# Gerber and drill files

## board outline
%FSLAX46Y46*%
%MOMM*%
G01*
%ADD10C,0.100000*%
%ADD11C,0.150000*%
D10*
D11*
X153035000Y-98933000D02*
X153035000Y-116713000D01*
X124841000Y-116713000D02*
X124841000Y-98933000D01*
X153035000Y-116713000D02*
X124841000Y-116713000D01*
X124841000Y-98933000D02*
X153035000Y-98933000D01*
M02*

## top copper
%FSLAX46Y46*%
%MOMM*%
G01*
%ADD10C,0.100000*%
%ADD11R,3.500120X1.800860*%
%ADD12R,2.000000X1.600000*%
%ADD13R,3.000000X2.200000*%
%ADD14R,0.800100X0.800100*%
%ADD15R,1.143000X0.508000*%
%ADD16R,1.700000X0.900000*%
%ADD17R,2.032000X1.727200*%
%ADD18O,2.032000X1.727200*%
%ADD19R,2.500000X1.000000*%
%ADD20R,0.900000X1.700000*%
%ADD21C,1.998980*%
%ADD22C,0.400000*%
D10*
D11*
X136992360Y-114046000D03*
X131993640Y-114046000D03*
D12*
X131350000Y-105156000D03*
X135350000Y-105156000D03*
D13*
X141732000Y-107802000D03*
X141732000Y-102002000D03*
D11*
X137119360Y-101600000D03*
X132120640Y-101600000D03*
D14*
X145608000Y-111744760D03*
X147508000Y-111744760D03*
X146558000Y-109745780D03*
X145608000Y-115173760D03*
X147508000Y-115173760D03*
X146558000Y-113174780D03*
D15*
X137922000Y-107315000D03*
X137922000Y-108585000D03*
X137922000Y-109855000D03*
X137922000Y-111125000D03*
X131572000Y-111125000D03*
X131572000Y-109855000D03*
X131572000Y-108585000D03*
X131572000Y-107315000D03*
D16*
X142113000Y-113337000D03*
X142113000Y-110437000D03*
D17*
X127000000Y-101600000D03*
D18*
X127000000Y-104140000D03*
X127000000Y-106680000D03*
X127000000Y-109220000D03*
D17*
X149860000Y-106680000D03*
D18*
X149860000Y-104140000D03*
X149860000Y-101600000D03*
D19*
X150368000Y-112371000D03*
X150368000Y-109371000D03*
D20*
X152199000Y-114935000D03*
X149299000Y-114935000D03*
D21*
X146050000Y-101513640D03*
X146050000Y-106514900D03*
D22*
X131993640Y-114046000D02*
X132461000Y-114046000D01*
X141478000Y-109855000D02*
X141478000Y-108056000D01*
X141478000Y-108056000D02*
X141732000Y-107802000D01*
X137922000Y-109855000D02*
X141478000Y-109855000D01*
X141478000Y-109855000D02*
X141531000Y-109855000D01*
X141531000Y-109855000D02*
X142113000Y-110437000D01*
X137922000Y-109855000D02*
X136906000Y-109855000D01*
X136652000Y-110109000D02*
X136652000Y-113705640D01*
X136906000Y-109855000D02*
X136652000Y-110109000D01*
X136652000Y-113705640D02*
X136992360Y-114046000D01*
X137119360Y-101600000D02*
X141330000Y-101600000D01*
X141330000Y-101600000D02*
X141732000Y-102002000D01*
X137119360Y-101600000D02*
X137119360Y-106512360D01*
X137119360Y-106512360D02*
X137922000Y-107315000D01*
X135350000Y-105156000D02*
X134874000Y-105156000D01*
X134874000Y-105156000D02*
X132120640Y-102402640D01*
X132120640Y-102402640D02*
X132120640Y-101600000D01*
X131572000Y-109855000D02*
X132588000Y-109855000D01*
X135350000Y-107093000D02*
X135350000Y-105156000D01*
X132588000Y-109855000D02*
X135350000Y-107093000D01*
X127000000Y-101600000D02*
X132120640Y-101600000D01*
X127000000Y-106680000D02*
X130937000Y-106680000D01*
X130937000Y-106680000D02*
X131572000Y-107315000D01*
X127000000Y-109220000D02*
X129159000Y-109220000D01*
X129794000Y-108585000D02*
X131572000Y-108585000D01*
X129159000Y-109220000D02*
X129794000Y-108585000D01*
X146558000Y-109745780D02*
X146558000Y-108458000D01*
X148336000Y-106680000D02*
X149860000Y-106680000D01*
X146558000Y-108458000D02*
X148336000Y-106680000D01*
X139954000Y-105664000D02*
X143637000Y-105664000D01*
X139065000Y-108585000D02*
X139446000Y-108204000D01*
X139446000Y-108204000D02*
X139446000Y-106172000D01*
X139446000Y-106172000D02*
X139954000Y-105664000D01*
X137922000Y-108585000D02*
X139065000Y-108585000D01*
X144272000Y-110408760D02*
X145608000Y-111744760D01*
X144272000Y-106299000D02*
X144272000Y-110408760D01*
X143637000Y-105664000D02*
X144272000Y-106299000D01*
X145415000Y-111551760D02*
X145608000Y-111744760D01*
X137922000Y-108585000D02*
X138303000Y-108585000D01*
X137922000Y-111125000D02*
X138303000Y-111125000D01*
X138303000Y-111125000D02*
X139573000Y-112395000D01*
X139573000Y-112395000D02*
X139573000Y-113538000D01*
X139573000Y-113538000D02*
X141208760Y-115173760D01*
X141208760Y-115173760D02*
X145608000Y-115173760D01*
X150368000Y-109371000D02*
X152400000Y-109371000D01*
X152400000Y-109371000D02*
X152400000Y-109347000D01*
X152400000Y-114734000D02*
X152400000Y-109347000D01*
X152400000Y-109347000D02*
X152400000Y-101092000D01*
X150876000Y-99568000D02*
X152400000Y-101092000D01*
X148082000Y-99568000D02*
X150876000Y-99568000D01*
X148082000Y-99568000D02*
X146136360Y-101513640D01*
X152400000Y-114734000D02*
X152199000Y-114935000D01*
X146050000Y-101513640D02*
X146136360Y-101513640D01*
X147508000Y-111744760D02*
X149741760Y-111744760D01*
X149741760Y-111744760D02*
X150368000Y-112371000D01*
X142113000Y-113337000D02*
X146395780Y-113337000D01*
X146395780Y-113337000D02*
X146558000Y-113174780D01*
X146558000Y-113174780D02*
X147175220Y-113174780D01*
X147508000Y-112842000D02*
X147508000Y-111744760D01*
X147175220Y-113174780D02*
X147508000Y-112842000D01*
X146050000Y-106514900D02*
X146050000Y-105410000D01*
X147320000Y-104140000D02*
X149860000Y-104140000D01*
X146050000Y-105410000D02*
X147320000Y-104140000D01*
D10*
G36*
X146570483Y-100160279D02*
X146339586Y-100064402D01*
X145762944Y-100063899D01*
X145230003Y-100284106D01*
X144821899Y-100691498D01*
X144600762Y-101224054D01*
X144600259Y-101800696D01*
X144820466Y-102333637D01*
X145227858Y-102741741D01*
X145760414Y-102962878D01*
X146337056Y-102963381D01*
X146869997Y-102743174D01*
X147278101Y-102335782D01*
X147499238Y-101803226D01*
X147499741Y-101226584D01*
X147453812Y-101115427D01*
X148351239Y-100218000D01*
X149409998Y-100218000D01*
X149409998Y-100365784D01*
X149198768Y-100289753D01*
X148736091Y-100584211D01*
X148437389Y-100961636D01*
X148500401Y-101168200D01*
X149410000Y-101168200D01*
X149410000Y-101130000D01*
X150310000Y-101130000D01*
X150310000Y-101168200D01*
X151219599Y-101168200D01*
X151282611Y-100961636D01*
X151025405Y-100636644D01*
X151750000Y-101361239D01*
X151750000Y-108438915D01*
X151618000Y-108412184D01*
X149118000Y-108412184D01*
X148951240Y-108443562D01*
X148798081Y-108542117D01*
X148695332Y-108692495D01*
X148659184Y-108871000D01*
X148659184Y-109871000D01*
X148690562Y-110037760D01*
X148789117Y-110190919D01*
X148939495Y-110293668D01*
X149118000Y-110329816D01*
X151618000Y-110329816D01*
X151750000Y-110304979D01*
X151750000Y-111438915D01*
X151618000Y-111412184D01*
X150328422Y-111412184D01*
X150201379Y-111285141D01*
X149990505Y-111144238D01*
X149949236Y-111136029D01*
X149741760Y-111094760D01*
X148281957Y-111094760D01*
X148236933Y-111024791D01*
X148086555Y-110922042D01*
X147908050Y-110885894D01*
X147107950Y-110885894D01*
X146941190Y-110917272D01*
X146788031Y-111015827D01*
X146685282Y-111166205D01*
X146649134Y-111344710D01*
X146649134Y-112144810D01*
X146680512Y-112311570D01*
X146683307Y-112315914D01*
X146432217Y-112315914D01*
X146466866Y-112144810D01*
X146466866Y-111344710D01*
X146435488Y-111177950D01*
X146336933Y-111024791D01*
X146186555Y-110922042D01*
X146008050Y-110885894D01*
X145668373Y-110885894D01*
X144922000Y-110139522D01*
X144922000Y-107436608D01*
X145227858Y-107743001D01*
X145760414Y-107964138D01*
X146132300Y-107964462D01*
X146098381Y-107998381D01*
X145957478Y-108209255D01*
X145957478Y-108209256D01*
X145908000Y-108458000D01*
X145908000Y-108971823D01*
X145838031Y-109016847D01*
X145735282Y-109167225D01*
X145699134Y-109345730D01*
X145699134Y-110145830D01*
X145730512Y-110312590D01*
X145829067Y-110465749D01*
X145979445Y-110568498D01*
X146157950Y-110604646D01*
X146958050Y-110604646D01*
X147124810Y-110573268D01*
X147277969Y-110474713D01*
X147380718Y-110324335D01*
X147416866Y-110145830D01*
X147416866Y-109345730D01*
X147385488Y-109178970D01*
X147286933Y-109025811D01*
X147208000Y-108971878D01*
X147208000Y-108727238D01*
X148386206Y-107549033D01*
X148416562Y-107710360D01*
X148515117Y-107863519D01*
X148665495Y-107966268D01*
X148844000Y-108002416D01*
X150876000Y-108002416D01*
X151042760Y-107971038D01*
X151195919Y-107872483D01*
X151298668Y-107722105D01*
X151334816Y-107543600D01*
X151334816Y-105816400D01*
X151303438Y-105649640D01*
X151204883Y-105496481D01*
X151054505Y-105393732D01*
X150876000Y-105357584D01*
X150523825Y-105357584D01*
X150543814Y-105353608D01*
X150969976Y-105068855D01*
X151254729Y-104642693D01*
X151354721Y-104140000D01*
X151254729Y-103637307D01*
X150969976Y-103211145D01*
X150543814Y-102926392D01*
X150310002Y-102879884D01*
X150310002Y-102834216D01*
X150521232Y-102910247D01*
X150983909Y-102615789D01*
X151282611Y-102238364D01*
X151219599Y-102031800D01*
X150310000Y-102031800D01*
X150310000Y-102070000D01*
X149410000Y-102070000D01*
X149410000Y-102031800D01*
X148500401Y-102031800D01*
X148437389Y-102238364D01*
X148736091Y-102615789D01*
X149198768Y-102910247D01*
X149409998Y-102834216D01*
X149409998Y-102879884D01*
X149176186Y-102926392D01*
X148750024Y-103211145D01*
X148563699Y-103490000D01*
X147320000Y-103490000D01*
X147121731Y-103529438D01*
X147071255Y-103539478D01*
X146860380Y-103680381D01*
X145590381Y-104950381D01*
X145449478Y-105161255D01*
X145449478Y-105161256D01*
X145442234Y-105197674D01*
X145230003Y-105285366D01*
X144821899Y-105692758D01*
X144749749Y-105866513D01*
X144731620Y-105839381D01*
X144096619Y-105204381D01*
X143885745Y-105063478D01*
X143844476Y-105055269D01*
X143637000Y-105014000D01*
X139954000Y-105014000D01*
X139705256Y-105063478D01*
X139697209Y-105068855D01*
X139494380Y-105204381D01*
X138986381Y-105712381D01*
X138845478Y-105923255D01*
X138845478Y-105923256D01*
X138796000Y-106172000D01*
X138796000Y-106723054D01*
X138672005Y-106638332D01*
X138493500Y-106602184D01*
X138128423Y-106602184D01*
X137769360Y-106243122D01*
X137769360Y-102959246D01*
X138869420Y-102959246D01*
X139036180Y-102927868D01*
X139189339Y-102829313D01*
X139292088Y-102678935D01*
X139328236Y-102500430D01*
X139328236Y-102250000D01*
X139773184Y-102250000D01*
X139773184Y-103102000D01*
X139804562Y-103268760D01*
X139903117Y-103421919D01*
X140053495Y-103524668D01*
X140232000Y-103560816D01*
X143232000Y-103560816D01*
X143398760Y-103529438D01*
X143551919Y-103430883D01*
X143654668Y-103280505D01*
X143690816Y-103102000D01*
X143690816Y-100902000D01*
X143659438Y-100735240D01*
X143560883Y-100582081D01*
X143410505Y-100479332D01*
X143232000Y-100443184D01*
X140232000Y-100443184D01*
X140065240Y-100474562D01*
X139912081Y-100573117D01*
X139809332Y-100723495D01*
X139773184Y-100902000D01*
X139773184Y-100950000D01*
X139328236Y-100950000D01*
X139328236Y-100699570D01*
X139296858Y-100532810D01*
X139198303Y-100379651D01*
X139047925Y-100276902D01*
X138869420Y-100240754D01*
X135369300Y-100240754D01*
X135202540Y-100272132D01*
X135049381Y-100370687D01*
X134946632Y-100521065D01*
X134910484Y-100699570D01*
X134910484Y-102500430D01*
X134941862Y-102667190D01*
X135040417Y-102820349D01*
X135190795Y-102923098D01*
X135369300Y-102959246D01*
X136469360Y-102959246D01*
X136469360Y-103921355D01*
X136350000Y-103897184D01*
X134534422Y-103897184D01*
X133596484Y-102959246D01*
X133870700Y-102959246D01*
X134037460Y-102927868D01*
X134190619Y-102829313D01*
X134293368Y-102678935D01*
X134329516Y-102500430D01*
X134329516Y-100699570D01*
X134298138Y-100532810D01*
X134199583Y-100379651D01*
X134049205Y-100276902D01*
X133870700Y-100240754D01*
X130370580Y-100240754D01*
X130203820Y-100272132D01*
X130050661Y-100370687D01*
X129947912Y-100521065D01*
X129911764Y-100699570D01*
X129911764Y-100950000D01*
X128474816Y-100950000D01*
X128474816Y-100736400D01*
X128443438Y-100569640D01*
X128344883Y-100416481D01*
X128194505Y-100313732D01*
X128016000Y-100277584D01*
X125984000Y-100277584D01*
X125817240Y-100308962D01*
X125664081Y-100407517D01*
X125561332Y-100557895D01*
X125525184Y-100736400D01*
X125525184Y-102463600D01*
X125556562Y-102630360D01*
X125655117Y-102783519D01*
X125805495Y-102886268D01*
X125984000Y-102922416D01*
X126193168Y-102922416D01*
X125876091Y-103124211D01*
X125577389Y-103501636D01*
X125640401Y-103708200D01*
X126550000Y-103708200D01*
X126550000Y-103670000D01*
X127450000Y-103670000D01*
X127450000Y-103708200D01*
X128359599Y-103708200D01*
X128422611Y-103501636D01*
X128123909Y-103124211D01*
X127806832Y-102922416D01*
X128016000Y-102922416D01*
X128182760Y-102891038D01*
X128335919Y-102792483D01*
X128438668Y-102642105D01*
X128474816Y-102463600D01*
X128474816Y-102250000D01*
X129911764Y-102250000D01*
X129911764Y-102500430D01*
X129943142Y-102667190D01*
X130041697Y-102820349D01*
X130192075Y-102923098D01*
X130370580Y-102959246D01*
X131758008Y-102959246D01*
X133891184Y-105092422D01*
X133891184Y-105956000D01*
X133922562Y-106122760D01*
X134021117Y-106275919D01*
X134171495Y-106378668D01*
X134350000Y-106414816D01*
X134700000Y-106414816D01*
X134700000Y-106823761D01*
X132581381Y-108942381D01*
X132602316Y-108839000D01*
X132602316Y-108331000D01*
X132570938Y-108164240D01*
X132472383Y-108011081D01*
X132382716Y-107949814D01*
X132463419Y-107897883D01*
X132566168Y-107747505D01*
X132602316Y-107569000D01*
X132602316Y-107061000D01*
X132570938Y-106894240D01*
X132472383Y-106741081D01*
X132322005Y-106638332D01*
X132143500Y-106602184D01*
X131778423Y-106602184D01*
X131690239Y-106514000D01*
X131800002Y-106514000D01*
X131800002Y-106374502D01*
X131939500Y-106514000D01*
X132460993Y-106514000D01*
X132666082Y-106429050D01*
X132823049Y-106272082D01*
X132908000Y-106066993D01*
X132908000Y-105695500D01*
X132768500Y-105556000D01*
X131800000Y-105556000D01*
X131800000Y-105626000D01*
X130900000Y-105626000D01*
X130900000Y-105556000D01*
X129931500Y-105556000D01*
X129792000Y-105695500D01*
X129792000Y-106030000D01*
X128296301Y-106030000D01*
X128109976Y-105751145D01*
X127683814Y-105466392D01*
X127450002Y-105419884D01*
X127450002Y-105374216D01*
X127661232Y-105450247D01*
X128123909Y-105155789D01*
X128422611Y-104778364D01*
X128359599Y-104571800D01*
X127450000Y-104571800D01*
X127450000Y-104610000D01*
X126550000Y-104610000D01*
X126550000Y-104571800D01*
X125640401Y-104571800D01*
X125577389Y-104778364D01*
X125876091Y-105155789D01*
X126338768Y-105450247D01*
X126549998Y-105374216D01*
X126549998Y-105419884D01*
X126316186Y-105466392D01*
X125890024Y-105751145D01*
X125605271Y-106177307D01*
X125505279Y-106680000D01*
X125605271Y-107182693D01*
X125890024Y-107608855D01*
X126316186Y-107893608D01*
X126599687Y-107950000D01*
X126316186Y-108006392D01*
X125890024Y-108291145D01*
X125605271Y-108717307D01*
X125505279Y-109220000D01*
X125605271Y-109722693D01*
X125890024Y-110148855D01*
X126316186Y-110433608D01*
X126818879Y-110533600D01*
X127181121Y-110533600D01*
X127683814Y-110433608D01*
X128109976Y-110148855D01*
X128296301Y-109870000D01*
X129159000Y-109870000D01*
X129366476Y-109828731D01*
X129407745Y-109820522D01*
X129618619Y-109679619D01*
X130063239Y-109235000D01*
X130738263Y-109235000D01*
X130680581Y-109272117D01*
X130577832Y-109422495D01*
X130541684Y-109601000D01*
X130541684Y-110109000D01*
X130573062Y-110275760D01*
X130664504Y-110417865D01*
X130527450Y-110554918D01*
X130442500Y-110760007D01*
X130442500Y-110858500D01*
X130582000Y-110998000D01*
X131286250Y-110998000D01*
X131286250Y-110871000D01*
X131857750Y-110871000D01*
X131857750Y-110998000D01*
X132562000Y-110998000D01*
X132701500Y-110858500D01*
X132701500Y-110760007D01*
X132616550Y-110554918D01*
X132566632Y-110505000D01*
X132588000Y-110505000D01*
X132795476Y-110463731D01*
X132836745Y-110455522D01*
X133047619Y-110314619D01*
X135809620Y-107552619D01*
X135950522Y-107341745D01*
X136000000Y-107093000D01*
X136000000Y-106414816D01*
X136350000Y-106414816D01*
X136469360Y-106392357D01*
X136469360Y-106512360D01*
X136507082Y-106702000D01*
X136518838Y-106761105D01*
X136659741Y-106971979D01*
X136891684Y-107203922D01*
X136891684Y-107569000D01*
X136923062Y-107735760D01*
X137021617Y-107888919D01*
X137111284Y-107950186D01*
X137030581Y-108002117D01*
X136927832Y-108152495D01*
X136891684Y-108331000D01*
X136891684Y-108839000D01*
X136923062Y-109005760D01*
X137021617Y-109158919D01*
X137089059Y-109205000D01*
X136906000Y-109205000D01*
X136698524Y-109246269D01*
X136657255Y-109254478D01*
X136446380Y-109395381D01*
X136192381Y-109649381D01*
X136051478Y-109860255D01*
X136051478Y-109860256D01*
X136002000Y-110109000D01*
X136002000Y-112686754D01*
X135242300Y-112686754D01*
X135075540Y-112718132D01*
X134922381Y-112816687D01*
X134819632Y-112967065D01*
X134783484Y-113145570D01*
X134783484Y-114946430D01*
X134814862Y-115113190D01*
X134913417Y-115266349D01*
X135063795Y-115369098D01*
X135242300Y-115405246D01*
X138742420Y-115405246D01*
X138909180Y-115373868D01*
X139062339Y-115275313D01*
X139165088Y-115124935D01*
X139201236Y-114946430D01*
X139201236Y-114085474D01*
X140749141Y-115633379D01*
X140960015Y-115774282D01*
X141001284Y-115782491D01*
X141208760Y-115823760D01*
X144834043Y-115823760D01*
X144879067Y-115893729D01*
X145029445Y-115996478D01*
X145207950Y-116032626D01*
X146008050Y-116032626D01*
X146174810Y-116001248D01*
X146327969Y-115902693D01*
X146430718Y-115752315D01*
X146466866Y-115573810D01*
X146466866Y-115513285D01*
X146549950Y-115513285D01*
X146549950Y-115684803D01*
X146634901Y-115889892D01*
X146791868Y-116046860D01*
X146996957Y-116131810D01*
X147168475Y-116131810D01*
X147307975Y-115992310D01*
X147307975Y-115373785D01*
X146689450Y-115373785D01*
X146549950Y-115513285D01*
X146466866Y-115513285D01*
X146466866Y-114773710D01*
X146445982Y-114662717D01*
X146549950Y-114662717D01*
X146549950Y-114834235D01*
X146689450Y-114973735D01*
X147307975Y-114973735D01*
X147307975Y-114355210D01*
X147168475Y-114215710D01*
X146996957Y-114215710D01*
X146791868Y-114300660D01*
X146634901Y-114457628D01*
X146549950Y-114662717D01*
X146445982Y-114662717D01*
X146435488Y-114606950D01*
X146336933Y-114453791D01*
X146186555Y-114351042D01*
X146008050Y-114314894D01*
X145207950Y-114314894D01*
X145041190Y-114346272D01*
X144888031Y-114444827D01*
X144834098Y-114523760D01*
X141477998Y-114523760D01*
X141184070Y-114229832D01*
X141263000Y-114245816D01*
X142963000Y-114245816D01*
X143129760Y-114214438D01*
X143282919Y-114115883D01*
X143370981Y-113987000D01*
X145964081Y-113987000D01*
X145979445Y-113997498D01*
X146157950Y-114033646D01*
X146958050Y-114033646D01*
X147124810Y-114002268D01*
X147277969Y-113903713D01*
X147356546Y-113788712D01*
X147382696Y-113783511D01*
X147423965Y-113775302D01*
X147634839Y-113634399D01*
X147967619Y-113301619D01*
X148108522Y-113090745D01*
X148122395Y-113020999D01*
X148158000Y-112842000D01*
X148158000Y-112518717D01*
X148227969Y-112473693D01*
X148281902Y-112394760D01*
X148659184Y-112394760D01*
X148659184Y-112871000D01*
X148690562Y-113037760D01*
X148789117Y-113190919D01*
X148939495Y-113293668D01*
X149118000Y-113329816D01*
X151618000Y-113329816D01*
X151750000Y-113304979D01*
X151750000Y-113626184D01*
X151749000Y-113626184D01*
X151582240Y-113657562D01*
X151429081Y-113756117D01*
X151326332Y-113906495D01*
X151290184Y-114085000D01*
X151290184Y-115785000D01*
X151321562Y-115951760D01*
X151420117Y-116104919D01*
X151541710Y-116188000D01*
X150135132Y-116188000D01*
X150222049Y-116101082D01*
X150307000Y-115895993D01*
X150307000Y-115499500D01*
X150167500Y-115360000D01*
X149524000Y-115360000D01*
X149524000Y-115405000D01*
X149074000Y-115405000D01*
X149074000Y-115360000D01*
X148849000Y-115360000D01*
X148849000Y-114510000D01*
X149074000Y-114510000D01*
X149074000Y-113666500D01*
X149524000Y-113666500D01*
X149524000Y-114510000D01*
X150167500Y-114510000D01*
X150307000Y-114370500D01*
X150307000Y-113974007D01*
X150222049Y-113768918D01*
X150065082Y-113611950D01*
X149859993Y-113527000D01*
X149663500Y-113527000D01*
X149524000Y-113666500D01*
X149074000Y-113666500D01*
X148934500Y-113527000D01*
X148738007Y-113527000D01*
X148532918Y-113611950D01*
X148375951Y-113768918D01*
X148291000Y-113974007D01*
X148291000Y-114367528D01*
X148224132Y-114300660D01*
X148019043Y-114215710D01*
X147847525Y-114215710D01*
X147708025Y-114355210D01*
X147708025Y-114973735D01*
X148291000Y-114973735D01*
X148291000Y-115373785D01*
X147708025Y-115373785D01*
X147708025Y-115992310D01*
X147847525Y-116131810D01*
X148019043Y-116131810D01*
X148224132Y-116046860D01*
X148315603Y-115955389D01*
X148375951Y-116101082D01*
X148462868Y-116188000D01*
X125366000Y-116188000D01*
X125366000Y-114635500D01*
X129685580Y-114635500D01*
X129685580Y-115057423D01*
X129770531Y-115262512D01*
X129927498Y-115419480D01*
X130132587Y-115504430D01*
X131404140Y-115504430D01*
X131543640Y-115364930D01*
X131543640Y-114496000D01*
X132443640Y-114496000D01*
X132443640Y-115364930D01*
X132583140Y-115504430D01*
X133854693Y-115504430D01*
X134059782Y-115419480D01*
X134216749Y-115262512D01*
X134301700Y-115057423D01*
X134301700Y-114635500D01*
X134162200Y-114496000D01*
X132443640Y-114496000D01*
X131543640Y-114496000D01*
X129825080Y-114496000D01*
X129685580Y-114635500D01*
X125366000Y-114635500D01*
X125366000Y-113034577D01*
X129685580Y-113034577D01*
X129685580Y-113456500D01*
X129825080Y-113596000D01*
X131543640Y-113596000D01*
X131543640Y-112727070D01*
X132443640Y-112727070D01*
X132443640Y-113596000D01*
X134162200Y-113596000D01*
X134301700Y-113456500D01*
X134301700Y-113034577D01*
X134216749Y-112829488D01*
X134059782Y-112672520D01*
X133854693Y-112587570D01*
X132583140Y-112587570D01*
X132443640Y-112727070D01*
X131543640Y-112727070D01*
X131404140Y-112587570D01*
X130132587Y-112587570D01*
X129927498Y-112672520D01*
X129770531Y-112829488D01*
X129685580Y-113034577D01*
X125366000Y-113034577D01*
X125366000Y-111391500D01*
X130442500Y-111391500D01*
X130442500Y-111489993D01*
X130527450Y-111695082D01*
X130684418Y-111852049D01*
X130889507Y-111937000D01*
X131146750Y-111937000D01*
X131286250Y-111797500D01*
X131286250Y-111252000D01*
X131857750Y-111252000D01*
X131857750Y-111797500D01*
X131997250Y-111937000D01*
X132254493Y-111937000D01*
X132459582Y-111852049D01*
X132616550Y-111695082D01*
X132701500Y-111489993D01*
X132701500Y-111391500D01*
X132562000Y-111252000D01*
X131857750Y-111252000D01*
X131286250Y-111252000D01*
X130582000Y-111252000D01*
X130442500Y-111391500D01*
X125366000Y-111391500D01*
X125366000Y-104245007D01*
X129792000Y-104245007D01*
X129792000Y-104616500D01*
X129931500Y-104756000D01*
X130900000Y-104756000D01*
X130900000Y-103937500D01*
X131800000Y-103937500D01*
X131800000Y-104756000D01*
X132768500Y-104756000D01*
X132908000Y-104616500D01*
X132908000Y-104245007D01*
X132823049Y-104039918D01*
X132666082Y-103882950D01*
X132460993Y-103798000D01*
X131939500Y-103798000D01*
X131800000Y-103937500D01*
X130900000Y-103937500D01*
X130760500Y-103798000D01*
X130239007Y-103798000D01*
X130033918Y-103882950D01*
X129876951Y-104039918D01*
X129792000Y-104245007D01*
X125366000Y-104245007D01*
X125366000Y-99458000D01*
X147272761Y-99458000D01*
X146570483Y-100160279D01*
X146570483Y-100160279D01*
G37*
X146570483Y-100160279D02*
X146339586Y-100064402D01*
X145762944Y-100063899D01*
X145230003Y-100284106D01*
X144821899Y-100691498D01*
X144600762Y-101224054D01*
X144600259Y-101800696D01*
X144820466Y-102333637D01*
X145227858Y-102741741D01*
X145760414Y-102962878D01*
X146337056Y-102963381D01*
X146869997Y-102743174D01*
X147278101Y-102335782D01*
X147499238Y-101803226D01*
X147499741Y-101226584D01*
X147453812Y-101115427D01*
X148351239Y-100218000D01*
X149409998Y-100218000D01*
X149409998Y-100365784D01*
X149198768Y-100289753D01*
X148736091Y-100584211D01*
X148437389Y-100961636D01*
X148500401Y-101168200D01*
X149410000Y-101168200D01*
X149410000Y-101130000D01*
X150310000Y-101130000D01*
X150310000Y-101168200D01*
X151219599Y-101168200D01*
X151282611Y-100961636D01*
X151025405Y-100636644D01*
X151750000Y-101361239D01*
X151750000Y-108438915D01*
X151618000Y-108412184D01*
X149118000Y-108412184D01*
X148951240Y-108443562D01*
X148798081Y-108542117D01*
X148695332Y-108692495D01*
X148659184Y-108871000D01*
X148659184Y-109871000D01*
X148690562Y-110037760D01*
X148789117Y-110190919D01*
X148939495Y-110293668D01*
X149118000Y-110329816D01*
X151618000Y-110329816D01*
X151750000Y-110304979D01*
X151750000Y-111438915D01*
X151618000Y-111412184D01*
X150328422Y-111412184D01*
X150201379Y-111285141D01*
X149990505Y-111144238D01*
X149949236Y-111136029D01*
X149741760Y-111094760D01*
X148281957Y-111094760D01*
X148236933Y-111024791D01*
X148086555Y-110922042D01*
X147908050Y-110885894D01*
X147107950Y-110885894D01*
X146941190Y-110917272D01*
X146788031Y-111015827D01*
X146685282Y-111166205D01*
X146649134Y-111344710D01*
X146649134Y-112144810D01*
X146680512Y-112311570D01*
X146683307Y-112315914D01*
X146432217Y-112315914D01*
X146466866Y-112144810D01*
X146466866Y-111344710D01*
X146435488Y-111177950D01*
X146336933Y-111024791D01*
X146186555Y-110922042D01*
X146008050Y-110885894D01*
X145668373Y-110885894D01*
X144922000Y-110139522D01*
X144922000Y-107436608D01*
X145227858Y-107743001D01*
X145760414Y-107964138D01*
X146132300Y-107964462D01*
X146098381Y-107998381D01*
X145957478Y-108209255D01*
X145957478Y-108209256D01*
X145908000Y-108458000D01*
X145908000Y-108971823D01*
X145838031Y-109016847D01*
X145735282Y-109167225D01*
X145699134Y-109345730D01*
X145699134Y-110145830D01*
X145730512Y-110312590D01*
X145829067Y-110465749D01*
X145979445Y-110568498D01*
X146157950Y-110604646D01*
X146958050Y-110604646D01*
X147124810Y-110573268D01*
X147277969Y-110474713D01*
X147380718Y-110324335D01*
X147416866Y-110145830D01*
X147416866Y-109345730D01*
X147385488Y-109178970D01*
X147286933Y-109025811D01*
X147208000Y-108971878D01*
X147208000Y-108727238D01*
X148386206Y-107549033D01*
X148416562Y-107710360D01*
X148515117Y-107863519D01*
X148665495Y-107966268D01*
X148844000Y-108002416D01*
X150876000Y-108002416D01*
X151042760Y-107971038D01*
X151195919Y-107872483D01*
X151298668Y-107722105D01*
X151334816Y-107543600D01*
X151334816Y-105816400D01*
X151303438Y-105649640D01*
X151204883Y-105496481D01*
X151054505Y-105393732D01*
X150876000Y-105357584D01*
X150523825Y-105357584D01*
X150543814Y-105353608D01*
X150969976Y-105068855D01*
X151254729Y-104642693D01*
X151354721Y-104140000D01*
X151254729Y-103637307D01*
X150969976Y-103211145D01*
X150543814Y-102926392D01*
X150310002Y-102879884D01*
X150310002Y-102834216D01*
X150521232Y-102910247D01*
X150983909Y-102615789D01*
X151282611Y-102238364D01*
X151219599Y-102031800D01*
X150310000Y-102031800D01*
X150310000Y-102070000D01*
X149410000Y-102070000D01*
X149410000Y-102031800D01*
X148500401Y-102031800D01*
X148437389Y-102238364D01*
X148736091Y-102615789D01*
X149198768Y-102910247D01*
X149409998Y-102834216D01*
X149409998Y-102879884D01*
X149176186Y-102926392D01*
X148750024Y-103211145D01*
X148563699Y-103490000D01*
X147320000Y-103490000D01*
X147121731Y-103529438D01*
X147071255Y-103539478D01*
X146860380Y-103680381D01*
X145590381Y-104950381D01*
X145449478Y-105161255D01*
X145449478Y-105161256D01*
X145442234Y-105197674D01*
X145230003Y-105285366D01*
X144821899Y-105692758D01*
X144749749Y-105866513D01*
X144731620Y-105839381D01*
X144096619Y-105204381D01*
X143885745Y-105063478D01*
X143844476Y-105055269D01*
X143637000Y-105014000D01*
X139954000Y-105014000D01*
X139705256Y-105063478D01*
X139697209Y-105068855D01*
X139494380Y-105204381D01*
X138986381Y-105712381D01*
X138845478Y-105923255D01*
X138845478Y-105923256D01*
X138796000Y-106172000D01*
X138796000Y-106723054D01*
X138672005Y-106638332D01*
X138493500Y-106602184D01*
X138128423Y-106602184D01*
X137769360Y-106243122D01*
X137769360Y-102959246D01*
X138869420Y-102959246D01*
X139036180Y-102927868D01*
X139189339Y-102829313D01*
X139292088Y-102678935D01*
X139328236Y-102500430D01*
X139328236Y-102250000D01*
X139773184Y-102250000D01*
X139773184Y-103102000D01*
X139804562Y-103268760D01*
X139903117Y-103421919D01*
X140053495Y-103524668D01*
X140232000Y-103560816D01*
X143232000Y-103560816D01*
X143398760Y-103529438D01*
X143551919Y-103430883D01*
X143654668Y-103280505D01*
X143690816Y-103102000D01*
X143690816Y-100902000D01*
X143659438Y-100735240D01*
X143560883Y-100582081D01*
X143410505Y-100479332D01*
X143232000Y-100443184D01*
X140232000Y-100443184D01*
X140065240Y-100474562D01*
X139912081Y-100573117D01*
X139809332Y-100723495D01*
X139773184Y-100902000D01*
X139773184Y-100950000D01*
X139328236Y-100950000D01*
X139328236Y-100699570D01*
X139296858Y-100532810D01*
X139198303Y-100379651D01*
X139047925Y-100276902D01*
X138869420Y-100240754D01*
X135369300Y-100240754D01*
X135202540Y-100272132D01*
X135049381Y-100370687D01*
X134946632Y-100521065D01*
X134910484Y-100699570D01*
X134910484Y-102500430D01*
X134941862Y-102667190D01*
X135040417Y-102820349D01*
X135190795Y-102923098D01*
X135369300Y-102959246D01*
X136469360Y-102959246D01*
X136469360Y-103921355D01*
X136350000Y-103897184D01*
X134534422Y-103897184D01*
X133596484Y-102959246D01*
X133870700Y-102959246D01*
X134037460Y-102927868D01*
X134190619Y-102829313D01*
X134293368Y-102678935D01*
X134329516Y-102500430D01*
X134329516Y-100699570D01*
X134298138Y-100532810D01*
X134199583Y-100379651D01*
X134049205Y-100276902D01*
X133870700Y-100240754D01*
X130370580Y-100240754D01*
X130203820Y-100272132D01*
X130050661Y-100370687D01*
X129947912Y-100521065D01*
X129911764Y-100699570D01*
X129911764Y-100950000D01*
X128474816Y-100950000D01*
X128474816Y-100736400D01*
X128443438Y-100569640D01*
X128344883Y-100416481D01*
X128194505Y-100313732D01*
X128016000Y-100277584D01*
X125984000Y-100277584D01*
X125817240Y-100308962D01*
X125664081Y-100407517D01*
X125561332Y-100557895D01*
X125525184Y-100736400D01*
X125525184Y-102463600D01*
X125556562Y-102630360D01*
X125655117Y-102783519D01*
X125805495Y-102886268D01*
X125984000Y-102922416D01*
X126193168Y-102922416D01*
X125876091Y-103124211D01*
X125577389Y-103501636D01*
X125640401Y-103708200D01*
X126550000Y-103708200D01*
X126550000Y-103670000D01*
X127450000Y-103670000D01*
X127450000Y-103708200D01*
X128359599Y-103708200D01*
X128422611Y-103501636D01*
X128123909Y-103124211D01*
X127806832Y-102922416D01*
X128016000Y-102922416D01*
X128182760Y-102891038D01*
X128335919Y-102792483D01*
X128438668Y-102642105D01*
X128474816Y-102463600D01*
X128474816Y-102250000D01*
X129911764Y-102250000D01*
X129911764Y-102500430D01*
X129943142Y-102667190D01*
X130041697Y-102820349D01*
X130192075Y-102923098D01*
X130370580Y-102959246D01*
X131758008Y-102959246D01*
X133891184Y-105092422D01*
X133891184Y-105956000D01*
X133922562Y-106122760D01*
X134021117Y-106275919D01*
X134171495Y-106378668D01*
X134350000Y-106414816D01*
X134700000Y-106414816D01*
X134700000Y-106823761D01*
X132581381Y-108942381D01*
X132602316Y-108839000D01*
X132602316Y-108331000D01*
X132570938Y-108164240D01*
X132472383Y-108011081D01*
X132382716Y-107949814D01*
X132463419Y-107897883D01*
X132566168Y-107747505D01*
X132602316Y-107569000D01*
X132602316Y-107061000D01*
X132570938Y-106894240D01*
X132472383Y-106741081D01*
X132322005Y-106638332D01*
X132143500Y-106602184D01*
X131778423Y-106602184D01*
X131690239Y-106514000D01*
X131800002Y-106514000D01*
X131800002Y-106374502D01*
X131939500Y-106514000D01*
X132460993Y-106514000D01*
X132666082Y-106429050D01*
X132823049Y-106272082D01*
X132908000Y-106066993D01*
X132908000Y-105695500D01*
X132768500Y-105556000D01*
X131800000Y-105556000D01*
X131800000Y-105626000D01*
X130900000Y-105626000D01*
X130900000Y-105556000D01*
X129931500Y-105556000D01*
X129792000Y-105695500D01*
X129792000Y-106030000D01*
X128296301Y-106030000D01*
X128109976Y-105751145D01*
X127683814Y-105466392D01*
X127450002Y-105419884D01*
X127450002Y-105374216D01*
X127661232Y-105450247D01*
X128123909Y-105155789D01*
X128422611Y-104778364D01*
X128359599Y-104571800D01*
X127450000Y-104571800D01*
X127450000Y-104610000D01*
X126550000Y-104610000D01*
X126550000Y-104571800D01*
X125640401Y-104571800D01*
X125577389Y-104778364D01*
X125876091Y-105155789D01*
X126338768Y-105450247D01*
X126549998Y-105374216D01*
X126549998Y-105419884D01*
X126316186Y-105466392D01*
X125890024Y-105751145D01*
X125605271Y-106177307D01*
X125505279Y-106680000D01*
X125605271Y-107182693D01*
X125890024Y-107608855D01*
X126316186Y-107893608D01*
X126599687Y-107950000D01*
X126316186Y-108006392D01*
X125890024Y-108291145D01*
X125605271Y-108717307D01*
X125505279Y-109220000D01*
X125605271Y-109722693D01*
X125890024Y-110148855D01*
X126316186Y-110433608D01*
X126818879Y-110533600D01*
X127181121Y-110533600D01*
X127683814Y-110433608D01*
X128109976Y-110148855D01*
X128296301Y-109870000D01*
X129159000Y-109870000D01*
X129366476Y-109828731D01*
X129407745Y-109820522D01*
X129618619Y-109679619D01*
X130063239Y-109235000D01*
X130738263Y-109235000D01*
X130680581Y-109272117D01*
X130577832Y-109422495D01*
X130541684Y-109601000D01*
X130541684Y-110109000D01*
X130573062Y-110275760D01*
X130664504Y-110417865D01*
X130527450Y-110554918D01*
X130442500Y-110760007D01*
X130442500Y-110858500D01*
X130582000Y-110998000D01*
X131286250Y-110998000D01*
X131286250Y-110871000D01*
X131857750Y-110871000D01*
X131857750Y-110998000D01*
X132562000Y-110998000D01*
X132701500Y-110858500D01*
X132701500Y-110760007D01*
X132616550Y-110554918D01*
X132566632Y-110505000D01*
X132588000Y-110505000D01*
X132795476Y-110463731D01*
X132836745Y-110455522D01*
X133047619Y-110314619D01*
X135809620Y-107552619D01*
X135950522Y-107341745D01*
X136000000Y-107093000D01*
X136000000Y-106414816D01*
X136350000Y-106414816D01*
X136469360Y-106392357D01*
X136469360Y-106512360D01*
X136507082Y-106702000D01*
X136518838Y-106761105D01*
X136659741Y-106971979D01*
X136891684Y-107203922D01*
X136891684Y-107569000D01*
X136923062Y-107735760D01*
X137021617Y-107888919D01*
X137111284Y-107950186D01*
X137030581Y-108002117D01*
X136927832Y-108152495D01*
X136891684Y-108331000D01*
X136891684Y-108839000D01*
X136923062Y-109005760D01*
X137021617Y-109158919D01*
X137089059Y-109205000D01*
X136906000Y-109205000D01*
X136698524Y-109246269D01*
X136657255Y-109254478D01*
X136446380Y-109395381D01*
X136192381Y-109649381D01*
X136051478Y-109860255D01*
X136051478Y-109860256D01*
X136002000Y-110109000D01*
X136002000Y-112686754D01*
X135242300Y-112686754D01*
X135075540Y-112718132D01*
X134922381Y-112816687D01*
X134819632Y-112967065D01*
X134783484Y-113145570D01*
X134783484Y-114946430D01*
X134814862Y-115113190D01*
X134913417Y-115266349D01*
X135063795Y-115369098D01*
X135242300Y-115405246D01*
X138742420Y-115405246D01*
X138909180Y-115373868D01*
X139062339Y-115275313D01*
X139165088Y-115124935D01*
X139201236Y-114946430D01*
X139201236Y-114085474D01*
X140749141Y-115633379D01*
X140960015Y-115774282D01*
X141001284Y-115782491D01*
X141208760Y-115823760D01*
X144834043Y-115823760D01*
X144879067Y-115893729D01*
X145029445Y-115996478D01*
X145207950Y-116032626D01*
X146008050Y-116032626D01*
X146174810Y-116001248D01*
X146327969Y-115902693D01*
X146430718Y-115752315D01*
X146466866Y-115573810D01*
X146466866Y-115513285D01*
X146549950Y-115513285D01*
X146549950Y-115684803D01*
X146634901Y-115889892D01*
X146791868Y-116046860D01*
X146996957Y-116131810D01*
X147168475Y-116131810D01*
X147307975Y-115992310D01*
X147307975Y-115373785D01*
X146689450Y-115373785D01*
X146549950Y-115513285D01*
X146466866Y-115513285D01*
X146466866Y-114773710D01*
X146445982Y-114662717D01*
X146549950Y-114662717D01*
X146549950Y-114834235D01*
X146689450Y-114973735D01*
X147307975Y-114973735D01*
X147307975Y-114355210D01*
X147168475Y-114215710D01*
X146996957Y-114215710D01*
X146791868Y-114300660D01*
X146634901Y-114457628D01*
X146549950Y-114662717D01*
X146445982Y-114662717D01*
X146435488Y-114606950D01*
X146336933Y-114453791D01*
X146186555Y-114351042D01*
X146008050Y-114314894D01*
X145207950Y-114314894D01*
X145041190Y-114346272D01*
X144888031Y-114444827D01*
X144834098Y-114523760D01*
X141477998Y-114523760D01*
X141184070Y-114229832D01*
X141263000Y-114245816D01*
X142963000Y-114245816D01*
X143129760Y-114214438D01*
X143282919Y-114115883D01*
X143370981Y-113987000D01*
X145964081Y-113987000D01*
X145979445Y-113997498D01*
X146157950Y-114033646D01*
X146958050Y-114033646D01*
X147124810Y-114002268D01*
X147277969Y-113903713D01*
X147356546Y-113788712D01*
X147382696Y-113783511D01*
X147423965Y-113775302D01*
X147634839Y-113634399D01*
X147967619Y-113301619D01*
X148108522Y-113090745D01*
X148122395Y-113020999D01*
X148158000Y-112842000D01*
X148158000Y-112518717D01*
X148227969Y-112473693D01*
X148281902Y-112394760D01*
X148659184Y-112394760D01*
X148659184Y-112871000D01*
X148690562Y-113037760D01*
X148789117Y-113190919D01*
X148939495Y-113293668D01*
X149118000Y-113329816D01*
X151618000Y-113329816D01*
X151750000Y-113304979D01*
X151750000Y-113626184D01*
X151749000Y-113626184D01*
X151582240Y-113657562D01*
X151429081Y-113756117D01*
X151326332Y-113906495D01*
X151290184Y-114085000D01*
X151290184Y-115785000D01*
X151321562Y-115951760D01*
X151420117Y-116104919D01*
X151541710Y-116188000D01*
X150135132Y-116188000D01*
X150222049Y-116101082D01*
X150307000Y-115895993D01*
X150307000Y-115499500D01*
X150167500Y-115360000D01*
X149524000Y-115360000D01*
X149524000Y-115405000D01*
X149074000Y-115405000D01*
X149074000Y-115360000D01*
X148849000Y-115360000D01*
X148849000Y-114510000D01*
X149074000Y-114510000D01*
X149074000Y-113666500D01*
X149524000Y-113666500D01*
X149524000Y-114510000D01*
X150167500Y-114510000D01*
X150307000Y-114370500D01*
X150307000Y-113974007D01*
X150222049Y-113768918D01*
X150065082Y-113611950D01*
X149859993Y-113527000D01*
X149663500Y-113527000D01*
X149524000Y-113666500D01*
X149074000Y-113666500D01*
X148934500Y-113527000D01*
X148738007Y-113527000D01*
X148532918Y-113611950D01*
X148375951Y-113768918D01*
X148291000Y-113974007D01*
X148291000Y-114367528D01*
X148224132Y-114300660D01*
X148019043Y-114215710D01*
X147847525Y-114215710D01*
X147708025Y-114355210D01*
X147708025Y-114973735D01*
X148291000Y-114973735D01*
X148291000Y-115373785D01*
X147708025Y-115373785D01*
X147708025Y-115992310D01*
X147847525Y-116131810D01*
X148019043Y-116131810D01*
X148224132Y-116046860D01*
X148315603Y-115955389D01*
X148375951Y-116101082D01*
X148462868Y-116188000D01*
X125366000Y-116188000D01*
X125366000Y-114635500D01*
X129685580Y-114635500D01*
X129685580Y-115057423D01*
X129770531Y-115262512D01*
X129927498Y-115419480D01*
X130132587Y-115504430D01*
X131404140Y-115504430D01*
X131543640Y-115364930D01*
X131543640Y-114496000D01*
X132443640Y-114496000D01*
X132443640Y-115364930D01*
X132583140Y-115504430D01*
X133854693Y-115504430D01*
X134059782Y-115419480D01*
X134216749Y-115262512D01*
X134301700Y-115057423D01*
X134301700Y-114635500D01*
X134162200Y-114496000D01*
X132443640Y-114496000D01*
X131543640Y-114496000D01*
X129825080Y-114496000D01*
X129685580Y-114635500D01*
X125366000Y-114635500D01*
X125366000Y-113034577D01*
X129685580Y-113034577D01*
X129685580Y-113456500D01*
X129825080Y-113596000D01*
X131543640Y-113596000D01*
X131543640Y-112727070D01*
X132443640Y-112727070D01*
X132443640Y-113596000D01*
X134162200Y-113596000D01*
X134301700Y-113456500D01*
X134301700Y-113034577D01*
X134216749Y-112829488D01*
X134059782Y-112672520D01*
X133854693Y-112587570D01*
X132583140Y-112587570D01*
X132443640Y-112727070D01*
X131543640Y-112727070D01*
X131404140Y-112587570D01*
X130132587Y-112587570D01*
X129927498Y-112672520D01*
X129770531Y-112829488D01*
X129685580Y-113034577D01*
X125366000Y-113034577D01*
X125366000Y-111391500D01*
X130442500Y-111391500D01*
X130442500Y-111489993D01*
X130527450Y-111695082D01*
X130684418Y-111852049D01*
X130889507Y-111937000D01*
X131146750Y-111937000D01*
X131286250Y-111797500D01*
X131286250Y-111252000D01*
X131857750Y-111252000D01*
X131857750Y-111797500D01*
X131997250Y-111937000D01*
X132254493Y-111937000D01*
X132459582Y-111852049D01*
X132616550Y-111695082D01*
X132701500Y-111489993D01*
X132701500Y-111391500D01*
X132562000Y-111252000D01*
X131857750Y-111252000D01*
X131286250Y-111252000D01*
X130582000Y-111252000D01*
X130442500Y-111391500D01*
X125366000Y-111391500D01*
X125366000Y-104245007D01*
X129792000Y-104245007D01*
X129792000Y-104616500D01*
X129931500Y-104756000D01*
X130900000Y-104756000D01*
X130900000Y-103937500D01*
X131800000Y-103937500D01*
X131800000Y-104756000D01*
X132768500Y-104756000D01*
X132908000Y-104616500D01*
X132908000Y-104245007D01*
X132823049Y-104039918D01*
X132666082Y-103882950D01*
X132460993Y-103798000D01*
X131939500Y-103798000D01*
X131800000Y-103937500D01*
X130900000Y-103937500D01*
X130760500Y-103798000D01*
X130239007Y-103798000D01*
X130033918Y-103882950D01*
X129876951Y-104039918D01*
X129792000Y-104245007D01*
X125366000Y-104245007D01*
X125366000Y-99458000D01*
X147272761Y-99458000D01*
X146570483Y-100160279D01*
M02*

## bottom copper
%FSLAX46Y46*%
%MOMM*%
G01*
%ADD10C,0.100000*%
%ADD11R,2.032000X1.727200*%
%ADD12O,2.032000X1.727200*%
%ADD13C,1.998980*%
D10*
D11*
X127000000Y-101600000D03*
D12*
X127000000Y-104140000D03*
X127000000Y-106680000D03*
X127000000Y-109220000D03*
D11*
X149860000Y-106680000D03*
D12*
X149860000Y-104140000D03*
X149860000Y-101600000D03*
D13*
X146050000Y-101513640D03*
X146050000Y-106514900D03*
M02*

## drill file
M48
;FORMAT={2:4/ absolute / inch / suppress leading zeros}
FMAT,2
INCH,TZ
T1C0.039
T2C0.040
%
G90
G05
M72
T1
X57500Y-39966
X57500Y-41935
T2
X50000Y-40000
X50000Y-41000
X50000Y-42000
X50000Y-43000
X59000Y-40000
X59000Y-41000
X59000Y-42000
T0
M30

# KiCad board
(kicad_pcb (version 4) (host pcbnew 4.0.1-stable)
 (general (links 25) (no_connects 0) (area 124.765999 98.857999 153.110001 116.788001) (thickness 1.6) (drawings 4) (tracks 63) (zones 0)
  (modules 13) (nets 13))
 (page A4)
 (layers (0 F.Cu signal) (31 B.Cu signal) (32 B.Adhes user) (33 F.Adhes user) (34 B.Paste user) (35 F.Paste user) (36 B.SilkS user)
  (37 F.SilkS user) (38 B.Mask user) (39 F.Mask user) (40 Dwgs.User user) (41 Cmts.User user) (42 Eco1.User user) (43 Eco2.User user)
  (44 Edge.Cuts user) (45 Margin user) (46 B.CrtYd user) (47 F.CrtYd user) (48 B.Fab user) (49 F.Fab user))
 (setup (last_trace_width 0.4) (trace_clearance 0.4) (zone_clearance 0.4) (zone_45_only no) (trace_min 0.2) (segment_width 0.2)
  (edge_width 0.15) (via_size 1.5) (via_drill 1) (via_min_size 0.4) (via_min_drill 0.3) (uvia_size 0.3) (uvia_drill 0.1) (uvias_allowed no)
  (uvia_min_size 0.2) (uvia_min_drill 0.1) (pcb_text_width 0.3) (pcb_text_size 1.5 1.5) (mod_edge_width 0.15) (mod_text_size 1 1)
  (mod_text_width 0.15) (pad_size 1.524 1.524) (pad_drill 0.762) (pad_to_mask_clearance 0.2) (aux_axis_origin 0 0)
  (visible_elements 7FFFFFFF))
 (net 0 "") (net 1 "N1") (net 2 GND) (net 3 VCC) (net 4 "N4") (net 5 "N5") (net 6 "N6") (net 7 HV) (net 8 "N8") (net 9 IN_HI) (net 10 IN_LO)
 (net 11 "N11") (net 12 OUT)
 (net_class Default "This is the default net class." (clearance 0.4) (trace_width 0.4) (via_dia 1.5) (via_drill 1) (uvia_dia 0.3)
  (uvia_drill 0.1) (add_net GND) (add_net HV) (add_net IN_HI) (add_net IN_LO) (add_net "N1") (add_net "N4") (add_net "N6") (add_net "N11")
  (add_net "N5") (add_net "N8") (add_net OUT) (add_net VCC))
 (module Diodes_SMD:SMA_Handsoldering (layer F.Cu) (at 134.493 114.046 180)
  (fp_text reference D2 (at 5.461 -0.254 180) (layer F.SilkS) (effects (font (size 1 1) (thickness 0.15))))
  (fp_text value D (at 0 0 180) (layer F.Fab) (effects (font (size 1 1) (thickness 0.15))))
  (pad 1 smd rect (at -2.49936 0 180) (size 3.50012 1.80086) (layers F.Cu F.Paste F.Mask) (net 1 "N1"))
  (pad 2 smd rect (at 2.49936 0 180) (size 3.50012 1.80086) (layers F.Cu F.Paste F.Mask) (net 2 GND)))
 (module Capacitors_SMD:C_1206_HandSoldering (layer F.Cu) (at 133.35 105.156)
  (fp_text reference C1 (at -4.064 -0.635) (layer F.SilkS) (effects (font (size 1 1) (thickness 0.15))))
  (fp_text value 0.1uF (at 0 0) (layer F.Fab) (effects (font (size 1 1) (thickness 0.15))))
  (pad 1 smd rect (at -2 0) (size 2 1.6) (layers F.Cu F.Paste F.Mask) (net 2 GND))
  (pad 2 smd rect (at 2 0) (size 2 1.6) (layers F.Cu F.Paste F.Mask) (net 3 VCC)))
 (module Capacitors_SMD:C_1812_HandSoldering (layer F.Cu) (at 141.732 104.902 90)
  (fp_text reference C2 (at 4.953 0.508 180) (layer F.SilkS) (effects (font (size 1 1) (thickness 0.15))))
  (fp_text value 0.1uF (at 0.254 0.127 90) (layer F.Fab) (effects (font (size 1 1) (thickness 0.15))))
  (pad 1 smd rect (at -2.9 0 90) (size 2.2 3) (layers F.Cu F.Paste F.Mask) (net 1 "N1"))
  (pad 2 smd rect (at 2.9 0 90) (size 2.2 3) (layers F.Cu F.Paste F.Mask) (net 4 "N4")))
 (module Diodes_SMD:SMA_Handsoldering (layer F.Cu) (at 134.62 101.6 180)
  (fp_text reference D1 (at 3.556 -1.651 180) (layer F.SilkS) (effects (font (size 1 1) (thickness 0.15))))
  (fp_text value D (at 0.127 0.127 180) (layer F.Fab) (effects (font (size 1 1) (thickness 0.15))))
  (pad 1 smd rect (at -2.49936 0 180) (size 3.50012 1.80086) (layers F.Cu F.Paste F.Mask) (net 4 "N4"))
  (pad 2 smd rect (at 2.49936 0 180) (size 3.50012 1.80086) (layers F.Cu F.Paste F.Mask) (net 3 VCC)))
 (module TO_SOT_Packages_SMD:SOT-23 (layer F.Cu) (at 146.558 110.744)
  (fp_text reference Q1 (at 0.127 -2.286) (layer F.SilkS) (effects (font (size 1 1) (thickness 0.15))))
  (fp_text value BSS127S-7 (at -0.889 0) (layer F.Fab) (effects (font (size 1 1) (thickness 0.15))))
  (pad 1 smd rect (at -0.95 1.00076) (size 0.8001 0.8001) (layers F.Cu F.Paste F.Mask) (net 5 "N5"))
  (pad 2 smd rect (at 0.95 1.00076) (size 0.8001 0.8001) (layers F.Cu F.Paste F.Mask) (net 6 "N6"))
  (pad 3 smd rect (at 0 -0.99822) (size 0.8001 0.8001) (layers F.Cu F.Paste F.Mask) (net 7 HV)))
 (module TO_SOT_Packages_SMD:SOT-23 (layer F.Cu) (at 146.558 114.173)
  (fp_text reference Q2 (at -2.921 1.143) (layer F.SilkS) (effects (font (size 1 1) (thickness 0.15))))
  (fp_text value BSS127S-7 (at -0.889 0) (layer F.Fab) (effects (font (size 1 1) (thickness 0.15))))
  (pad 1 smd rect (at -0.95 1.00076) (size 0.8001 0.8001) (layers F.Cu F.Paste F.Mask) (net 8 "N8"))
  (pad 2 smd rect (at 0.95 1.00076) (size 0.8001 0.8001) (layers F.Cu F.Paste F.Mask) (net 2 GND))
  (pad 3 smd rect (at 0 -0.99822) (size 0.8001 0.8001) (layers F.Cu F.Paste F.Mask) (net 6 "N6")))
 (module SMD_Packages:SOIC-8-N (layer F.Cu) (at 134.747 109.22 270)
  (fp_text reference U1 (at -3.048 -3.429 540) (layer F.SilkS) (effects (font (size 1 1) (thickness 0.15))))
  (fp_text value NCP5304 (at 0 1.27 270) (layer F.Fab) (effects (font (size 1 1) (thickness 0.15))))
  (pad 8 smd rect (at -1.905 -3.175 270) (size 0.508 1.143) (layers F.Cu F.Paste F.Mask) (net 4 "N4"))
  (pad 7 smd rect (at -0.635 -3.175 270) (size 0.508 1.143) (layers F.Cu F.Paste F.Mask) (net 5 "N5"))
  (pad 6 smd rect (at 0.635 -3.175 270) (size 0.508 1.143) (layers F.Cu F.Paste F.Mask) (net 1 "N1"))
  (pad 5 smd rect (at 1.905 -3.175 270) (size 0.508 1.143) (layers F.Cu F.Paste F.Mask) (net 8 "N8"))
  (pad 4 smd rect (at 1.905 3.175 270) (size 0.508 1.143) (layers F.Cu F.Paste F.Mask) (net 2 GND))
  (pad 3 smd rect (at 0.635 3.175 270) (size 0.508 1.143) (layers F.Cu F.Paste F.Mask) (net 3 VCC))
  (pad 2 smd rect (at -0.635 3.175 270) (size 0.508 1.143) (layers F.Cu F.Paste F.Mask) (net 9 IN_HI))
  (pad 1 smd rect (at -1.905 3.175 270) (size 0.508 1.143) (layers F.Cu F.Paste F.Mask) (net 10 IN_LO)))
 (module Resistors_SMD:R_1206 (layer F.Cu) (at 142.113 111.887 90)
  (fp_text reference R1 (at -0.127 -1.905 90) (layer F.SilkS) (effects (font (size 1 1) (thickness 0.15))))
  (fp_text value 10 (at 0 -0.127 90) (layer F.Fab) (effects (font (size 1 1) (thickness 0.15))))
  (pad 1 smd rect (at -1.45 0 90) (size 0.9 1.7) (layers F.Cu F.Paste F.Mask) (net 6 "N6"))
  (pad 2 smd rect (at 1.45 0 90) (size 0.9 1.7) (layers F.Cu F.Paste F.Mask) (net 1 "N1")))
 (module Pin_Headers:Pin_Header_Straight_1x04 (layer F.Cu) (at 127 101.6)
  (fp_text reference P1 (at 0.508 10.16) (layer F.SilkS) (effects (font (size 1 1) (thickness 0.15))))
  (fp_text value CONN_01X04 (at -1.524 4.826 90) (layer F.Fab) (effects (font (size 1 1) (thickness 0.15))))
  (pad 1 thru_hole rect (at 0 0) (size 2.032 1.7272) (drill 1.016) (layers *.Cu *.Mask F.SilkS) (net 3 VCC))
  (pad 2 thru_hole oval (at 0 2.54) (size 2.032 1.7272) (drill 1.016) (layers *.Cu *.Mask F.SilkS) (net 2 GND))
  (pad 3 thru_hole oval (at 0 5.08) (size 2.032 1.7272) (drill 1.016) (layers *.Cu *.Mask F.SilkS) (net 10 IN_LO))
  (pad 4 thru_hole oval (at 0 7.62) (size 2.032 1.7272) (drill 1.016) (layers *.Cu *.Mask F.SilkS) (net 9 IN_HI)))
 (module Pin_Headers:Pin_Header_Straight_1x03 (layer F.Cu) (at 149.86 106.68 180)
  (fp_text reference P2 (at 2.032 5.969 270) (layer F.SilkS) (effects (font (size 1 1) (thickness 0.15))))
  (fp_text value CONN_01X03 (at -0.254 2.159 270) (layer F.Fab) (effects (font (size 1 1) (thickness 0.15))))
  (pad 1 thru_hole rect (at 0 0 180) (size 2.032 1.7272) (drill 1.016) (layers *.Cu *.Mask F.SilkS) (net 7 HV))
  (pad 2 thru_hole oval (at 0 2.54 180) (size 2.032 1.7272) (drill 1.016) (layers *.Cu *.Mask F.SilkS) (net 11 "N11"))
  (pad 3 thru_hole oval (at 0 5.08 180) (size 2.032 1.7272) (drill 1.016) (layers *.Cu *.Mask F.SilkS) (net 2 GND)))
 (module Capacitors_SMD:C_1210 (layer F.Cu) (at 150.368 110.871 90)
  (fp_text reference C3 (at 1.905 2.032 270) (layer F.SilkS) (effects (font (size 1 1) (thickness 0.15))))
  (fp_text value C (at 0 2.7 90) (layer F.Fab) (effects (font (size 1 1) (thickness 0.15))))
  (pad 1 smd rect (at -1.5 0 90) (size 1 2.5) (layers F.Cu F.Paste F.Mask) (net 6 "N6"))
  (pad 2 smd rect (at 1.5 0 90) (size 1 2.5) (layers F.Cu F.Paste F.Mask) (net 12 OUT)))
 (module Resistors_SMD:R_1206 (layer F.Cu) (at 150.749 114.935 180)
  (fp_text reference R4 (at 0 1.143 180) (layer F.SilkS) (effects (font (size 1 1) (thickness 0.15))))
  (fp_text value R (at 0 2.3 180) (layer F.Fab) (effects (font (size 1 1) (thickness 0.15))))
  (pad 1 smd rect (at -1.45 0 180) (size 0.9 1.7) (layers F.Cu F.Paste F.Mask) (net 12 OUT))
  (pad 2 smd rect (at 1.45 0 180) (size 0.9 1.7) (layers F.Cu F.Paste F.Mask) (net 2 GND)))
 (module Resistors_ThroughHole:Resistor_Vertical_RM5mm (layer F.Cu) (at 146.05 104.013 270)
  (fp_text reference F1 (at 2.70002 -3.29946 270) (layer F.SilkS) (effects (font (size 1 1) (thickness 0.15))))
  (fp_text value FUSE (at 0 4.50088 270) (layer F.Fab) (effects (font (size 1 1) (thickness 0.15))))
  (pad 1 thru_hole circle (at -2.49936 0 270) (size 1.99898 1.99898) (drill 1.00076) (layers *.Cu *.SilkS *.Mask) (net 12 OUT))
  (pad 2 thru_hole circle (at 2.5019 0 270) (size 1.99898 1.99898) (drill 1.00076) (layers *.Cu *.SilkS *.Mask) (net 11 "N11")))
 (gr_line (start 153.035 98.933) (end 153.035 116.713) (angle 90) (layer Edge.Cuts) (width 0.15))
 (gr_line (start 124.841 116.713) (end 124.841 98.933) (angle 90) (layer Edge.Cuts) (width 0.15))
 (gr_line (start 153.035 116.713) (end 124.841 116.713) (angle 90) (layer Edge.Cuts) (width 0.15))
 (gr_line (start 124.841 98.933) (end 153.035 98.933) (angle 90) (layer Edge.Cuts) (width 0.15))
 (segment (start 131.99364 114.046) (end 132.461 114.046) (width 0.4) (layer F.Cu) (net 2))
 (segment (start 141.478 109.855) (end 141.478 108.056) (width 0.4) (layer F.Cu) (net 1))
 (segment (start 141.478 108.056) (end 141.732 107.802) (width 0.4) (layer F.Cu) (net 1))
 (segment (start 137.922 109.855) (end 141.478 109.855) (width 0.4) (layer F.Cu) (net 1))
 (segment (start 141.478 109.855) (end 141.531 109.855) (width 0.4) (layer F.Cu) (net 1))
 (segment (start 141.531 109.855) (end 142.113 110.437) (width 0.4) (layer F.Cu) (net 1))
 (segment (start 137.922 109.855) (end 136.906 109.855) (width 0.4) (layer F.Cu) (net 1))
 (segment (start 136.652 110.109) (end 136.652 113.70564) (width 0.4) (layer F.Cu) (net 1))
 (segment (start 136.906 109.855) (end 136.652 110.109) (width 0.4) (layer F.Cu) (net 1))
 (segment (start 136.652 113.70564) (end 136.99236 114.046) (width 0.4) (layer F.Cu) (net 1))
 (segment (start 137.11936 101.6) (end 141.33 101.6) (width 0.4) (layer F.Cu) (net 4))
 (segment (start 141.33 101.6) (end 141.732 102.002) (width 0.4) (layer F.Cu) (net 4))
 (segment (start 137.11936 101.6) (end 137.11936 106.51236) (width 0.4) (layer F.Cu) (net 4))
 (segment (start 137.11936 106.51236) (end 137.922 107.315) (width 0.4) (layer F.Cu) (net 4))
 (segment (start 135.35 105.156) (end 134.874 105.156) (width 0.4) (layer F.Cu) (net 3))
 (segment (start 134.874 105.156) (end 132.12064 102.40264) (width 0.4) (layer F.Cu) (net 3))
 (segment (start 132.12064 102.40264) (end 132.12064 101.6) (width 0.4) (layer F.Cu) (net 3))
 (segment (start 131.572 109.855) (end 132.588 109.855) (width 0.4) (layer F.Cu) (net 3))
 (segment (start 135.35 107.093) (end 135.35 105.156) (width 0.4) (layer F.Cu) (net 3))
 (segment (start 132.588 109.855) (end 135.35 107.093) (width 0.4) (layer F.Cu) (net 3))
 (segment (start 127 101.6) (end 132.12064 101.6) (width 0.4) (layer F.Cu) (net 3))
 (segment (start 127 106.68) (end 130.937 106.68) (width 0.4) (layer F.Cu) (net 10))
 (segment (start 130.937 106.68) (end 131.572 107.315) (width 0.4) (layer F.Cu) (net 10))
 (segment (start 127 109.22) (end 129.159 109.22) (width 0.4) (layer F.Cu) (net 9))
 (segment (start 129.794 108.585) (end 131.572 108.585) (width 0.4) (layer F.Cu) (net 9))
 (segment (start 129.159 109.22) (end 129.794 108.585) (width 0.4) (layer F.Cu) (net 9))
 (segment (start 146.558 109.74578) (end 146.558 108.458) (width 0.4) (layer F.Cu) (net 7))
 (segment (start 148.336 106.68) (end 149.86 106.68) (width 0.4) (layer F.Cu) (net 7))
 (segment (start 146.558 108.458) (end 148.336 106.68) (width 0.4) (layer F.Cu) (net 7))
 (segment (start 139.954 105.664) (end 143.637 105.664) (width 0.4) (layer F.Cu) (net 5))
 (segment (start 139.065 108.585) (end 139.446 108.204) (width 0.4) (layer F.Cu) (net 5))
 (segment (start 139.446 108.204) (end 139.446 106.172) (width 0.4) (layer F.Cu) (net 5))
 (segment (start 139.446 106.172) (end 139.954 105.664) (width 0.4) (layer F.Cu) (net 5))
 (segment (start 137.922 108.585) (end 139.065 108.585) (width 0.4) (layer F.Cu) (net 5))
 (segment (start 144.272 110.40876) (end 145.608 111.74476) (width 0.4) (layer F.Cu) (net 5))
 (segment (start 144.272 106.299) (end 144.272 110.40876) (width 0.4) (layer F.Cu) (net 5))
 (segment (start 143.637 105.664) (end 144.272 106.299) (width 0.4) (layer F.Cu) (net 5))
 (segment (start 145.415 111.55176) (end 145.608 111.74476) (width 0.4) (layer F.Cu) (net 5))
 (segment (start 137.922 108.585) (end 138.303 108.585) (width 0.4) (layer F.Cu) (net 5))
 (segment (start 137.922 111.125) (end 138.303 111.125) (width 0.4) (layer F.Cu) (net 8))
 (segment (start 138.303 111.125) (end 139.573 112.395) (width 0.4) (layer F.Cu) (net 8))
 (segment (start 139.573 112.395) (end 139.573 113.538) (width 0.4) (layer F.Cu) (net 8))
 (segment (start 139.573 113.538) (end 141.20876 115.17376) (width 0.4) (layer F.Cu) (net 8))
 (segment (start 141.20876 115.17376) (end 145.608 115.17376) (width 0.4) (layer F.Cu) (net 8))
 (segment (start 150.368 109.371) (end 152.4 109.371) (width 0.4) (layer F.Cu) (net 12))
 (segment (start 152.4 109.371) (end 152.4 109.347) (width 0.4) (layer F.Cu) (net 12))
 (segment (start 152.4 114.734) (end 152.4 109.347) (width 0.4) (layer F.Cu) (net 12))
 (segment (start 152.4 109.347) (end 152.4 101.092) (width 0.4) (layer F.Cu) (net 12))
 (segment (start 150.876 99.568) (end 152.4 101.092) (width 0.4) (layer F.Cu) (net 12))
 (segment (start 148.082 99.568) (end 150.876 99.568) (width 0.4) (layer F.Cu) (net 12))
 (segment (start 148.082 99.568) (end 146.13636 101.51364) (width 0.4) (layer F.Cu) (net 12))
 (segment (start 152.4 114.734) (end 152.199 114.935) (width 0.4) (layer F.Cu) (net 12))
 (segment (start 146.05 101.51364) (end 146.13636 101.51364) (width 0.4) (layer F.Cu) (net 12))
 (segment (start 147.508 111.74476) (end 149.74176 111.74476) (width 0.4) (layer F.Cu) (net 6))
 (segment (start 149.74176 111.74476) (end 150.368 112.371) (width 0.4) (layer F.Cu) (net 6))
 (segment (start 142.113 113.337) (end 146.39578 113.337) (width 0.4) (layer F.Cu) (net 6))
 (segment (start 146.39578 113.337) (end 146.558 113.17478) (width 0.4) (layer F.Cu) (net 6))
 (segment (start 146.558 113.17478) (end 147.17522 113.17478) (width 0.4) (layer F.Cu) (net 6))
 (segment (start 147.508 112.842) (end 147.508 111.74476) (width 0.4) (layer F.Cu) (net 6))
 (segment (start 147.17522 113.17478) (end 147.508 112.842) (width 0.4) (layer F.Cu) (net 6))
 (segment (start 146.05 106.5149) (end 146.05 105.41) (width 0.4) (layer F.Cu) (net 11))
 (segment (start 147.32 104.14) (end 149.86 104.14) (width 0.4) (layer F.Cu) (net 11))
 (segment (start 146.05 105.41) (end 147.32 104.14) (width 0.4) (layer F.Cu) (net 11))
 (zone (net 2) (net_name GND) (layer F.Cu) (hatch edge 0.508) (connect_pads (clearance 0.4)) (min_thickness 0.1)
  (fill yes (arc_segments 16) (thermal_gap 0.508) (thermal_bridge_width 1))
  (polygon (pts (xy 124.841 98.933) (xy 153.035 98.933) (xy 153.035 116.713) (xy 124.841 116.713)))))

